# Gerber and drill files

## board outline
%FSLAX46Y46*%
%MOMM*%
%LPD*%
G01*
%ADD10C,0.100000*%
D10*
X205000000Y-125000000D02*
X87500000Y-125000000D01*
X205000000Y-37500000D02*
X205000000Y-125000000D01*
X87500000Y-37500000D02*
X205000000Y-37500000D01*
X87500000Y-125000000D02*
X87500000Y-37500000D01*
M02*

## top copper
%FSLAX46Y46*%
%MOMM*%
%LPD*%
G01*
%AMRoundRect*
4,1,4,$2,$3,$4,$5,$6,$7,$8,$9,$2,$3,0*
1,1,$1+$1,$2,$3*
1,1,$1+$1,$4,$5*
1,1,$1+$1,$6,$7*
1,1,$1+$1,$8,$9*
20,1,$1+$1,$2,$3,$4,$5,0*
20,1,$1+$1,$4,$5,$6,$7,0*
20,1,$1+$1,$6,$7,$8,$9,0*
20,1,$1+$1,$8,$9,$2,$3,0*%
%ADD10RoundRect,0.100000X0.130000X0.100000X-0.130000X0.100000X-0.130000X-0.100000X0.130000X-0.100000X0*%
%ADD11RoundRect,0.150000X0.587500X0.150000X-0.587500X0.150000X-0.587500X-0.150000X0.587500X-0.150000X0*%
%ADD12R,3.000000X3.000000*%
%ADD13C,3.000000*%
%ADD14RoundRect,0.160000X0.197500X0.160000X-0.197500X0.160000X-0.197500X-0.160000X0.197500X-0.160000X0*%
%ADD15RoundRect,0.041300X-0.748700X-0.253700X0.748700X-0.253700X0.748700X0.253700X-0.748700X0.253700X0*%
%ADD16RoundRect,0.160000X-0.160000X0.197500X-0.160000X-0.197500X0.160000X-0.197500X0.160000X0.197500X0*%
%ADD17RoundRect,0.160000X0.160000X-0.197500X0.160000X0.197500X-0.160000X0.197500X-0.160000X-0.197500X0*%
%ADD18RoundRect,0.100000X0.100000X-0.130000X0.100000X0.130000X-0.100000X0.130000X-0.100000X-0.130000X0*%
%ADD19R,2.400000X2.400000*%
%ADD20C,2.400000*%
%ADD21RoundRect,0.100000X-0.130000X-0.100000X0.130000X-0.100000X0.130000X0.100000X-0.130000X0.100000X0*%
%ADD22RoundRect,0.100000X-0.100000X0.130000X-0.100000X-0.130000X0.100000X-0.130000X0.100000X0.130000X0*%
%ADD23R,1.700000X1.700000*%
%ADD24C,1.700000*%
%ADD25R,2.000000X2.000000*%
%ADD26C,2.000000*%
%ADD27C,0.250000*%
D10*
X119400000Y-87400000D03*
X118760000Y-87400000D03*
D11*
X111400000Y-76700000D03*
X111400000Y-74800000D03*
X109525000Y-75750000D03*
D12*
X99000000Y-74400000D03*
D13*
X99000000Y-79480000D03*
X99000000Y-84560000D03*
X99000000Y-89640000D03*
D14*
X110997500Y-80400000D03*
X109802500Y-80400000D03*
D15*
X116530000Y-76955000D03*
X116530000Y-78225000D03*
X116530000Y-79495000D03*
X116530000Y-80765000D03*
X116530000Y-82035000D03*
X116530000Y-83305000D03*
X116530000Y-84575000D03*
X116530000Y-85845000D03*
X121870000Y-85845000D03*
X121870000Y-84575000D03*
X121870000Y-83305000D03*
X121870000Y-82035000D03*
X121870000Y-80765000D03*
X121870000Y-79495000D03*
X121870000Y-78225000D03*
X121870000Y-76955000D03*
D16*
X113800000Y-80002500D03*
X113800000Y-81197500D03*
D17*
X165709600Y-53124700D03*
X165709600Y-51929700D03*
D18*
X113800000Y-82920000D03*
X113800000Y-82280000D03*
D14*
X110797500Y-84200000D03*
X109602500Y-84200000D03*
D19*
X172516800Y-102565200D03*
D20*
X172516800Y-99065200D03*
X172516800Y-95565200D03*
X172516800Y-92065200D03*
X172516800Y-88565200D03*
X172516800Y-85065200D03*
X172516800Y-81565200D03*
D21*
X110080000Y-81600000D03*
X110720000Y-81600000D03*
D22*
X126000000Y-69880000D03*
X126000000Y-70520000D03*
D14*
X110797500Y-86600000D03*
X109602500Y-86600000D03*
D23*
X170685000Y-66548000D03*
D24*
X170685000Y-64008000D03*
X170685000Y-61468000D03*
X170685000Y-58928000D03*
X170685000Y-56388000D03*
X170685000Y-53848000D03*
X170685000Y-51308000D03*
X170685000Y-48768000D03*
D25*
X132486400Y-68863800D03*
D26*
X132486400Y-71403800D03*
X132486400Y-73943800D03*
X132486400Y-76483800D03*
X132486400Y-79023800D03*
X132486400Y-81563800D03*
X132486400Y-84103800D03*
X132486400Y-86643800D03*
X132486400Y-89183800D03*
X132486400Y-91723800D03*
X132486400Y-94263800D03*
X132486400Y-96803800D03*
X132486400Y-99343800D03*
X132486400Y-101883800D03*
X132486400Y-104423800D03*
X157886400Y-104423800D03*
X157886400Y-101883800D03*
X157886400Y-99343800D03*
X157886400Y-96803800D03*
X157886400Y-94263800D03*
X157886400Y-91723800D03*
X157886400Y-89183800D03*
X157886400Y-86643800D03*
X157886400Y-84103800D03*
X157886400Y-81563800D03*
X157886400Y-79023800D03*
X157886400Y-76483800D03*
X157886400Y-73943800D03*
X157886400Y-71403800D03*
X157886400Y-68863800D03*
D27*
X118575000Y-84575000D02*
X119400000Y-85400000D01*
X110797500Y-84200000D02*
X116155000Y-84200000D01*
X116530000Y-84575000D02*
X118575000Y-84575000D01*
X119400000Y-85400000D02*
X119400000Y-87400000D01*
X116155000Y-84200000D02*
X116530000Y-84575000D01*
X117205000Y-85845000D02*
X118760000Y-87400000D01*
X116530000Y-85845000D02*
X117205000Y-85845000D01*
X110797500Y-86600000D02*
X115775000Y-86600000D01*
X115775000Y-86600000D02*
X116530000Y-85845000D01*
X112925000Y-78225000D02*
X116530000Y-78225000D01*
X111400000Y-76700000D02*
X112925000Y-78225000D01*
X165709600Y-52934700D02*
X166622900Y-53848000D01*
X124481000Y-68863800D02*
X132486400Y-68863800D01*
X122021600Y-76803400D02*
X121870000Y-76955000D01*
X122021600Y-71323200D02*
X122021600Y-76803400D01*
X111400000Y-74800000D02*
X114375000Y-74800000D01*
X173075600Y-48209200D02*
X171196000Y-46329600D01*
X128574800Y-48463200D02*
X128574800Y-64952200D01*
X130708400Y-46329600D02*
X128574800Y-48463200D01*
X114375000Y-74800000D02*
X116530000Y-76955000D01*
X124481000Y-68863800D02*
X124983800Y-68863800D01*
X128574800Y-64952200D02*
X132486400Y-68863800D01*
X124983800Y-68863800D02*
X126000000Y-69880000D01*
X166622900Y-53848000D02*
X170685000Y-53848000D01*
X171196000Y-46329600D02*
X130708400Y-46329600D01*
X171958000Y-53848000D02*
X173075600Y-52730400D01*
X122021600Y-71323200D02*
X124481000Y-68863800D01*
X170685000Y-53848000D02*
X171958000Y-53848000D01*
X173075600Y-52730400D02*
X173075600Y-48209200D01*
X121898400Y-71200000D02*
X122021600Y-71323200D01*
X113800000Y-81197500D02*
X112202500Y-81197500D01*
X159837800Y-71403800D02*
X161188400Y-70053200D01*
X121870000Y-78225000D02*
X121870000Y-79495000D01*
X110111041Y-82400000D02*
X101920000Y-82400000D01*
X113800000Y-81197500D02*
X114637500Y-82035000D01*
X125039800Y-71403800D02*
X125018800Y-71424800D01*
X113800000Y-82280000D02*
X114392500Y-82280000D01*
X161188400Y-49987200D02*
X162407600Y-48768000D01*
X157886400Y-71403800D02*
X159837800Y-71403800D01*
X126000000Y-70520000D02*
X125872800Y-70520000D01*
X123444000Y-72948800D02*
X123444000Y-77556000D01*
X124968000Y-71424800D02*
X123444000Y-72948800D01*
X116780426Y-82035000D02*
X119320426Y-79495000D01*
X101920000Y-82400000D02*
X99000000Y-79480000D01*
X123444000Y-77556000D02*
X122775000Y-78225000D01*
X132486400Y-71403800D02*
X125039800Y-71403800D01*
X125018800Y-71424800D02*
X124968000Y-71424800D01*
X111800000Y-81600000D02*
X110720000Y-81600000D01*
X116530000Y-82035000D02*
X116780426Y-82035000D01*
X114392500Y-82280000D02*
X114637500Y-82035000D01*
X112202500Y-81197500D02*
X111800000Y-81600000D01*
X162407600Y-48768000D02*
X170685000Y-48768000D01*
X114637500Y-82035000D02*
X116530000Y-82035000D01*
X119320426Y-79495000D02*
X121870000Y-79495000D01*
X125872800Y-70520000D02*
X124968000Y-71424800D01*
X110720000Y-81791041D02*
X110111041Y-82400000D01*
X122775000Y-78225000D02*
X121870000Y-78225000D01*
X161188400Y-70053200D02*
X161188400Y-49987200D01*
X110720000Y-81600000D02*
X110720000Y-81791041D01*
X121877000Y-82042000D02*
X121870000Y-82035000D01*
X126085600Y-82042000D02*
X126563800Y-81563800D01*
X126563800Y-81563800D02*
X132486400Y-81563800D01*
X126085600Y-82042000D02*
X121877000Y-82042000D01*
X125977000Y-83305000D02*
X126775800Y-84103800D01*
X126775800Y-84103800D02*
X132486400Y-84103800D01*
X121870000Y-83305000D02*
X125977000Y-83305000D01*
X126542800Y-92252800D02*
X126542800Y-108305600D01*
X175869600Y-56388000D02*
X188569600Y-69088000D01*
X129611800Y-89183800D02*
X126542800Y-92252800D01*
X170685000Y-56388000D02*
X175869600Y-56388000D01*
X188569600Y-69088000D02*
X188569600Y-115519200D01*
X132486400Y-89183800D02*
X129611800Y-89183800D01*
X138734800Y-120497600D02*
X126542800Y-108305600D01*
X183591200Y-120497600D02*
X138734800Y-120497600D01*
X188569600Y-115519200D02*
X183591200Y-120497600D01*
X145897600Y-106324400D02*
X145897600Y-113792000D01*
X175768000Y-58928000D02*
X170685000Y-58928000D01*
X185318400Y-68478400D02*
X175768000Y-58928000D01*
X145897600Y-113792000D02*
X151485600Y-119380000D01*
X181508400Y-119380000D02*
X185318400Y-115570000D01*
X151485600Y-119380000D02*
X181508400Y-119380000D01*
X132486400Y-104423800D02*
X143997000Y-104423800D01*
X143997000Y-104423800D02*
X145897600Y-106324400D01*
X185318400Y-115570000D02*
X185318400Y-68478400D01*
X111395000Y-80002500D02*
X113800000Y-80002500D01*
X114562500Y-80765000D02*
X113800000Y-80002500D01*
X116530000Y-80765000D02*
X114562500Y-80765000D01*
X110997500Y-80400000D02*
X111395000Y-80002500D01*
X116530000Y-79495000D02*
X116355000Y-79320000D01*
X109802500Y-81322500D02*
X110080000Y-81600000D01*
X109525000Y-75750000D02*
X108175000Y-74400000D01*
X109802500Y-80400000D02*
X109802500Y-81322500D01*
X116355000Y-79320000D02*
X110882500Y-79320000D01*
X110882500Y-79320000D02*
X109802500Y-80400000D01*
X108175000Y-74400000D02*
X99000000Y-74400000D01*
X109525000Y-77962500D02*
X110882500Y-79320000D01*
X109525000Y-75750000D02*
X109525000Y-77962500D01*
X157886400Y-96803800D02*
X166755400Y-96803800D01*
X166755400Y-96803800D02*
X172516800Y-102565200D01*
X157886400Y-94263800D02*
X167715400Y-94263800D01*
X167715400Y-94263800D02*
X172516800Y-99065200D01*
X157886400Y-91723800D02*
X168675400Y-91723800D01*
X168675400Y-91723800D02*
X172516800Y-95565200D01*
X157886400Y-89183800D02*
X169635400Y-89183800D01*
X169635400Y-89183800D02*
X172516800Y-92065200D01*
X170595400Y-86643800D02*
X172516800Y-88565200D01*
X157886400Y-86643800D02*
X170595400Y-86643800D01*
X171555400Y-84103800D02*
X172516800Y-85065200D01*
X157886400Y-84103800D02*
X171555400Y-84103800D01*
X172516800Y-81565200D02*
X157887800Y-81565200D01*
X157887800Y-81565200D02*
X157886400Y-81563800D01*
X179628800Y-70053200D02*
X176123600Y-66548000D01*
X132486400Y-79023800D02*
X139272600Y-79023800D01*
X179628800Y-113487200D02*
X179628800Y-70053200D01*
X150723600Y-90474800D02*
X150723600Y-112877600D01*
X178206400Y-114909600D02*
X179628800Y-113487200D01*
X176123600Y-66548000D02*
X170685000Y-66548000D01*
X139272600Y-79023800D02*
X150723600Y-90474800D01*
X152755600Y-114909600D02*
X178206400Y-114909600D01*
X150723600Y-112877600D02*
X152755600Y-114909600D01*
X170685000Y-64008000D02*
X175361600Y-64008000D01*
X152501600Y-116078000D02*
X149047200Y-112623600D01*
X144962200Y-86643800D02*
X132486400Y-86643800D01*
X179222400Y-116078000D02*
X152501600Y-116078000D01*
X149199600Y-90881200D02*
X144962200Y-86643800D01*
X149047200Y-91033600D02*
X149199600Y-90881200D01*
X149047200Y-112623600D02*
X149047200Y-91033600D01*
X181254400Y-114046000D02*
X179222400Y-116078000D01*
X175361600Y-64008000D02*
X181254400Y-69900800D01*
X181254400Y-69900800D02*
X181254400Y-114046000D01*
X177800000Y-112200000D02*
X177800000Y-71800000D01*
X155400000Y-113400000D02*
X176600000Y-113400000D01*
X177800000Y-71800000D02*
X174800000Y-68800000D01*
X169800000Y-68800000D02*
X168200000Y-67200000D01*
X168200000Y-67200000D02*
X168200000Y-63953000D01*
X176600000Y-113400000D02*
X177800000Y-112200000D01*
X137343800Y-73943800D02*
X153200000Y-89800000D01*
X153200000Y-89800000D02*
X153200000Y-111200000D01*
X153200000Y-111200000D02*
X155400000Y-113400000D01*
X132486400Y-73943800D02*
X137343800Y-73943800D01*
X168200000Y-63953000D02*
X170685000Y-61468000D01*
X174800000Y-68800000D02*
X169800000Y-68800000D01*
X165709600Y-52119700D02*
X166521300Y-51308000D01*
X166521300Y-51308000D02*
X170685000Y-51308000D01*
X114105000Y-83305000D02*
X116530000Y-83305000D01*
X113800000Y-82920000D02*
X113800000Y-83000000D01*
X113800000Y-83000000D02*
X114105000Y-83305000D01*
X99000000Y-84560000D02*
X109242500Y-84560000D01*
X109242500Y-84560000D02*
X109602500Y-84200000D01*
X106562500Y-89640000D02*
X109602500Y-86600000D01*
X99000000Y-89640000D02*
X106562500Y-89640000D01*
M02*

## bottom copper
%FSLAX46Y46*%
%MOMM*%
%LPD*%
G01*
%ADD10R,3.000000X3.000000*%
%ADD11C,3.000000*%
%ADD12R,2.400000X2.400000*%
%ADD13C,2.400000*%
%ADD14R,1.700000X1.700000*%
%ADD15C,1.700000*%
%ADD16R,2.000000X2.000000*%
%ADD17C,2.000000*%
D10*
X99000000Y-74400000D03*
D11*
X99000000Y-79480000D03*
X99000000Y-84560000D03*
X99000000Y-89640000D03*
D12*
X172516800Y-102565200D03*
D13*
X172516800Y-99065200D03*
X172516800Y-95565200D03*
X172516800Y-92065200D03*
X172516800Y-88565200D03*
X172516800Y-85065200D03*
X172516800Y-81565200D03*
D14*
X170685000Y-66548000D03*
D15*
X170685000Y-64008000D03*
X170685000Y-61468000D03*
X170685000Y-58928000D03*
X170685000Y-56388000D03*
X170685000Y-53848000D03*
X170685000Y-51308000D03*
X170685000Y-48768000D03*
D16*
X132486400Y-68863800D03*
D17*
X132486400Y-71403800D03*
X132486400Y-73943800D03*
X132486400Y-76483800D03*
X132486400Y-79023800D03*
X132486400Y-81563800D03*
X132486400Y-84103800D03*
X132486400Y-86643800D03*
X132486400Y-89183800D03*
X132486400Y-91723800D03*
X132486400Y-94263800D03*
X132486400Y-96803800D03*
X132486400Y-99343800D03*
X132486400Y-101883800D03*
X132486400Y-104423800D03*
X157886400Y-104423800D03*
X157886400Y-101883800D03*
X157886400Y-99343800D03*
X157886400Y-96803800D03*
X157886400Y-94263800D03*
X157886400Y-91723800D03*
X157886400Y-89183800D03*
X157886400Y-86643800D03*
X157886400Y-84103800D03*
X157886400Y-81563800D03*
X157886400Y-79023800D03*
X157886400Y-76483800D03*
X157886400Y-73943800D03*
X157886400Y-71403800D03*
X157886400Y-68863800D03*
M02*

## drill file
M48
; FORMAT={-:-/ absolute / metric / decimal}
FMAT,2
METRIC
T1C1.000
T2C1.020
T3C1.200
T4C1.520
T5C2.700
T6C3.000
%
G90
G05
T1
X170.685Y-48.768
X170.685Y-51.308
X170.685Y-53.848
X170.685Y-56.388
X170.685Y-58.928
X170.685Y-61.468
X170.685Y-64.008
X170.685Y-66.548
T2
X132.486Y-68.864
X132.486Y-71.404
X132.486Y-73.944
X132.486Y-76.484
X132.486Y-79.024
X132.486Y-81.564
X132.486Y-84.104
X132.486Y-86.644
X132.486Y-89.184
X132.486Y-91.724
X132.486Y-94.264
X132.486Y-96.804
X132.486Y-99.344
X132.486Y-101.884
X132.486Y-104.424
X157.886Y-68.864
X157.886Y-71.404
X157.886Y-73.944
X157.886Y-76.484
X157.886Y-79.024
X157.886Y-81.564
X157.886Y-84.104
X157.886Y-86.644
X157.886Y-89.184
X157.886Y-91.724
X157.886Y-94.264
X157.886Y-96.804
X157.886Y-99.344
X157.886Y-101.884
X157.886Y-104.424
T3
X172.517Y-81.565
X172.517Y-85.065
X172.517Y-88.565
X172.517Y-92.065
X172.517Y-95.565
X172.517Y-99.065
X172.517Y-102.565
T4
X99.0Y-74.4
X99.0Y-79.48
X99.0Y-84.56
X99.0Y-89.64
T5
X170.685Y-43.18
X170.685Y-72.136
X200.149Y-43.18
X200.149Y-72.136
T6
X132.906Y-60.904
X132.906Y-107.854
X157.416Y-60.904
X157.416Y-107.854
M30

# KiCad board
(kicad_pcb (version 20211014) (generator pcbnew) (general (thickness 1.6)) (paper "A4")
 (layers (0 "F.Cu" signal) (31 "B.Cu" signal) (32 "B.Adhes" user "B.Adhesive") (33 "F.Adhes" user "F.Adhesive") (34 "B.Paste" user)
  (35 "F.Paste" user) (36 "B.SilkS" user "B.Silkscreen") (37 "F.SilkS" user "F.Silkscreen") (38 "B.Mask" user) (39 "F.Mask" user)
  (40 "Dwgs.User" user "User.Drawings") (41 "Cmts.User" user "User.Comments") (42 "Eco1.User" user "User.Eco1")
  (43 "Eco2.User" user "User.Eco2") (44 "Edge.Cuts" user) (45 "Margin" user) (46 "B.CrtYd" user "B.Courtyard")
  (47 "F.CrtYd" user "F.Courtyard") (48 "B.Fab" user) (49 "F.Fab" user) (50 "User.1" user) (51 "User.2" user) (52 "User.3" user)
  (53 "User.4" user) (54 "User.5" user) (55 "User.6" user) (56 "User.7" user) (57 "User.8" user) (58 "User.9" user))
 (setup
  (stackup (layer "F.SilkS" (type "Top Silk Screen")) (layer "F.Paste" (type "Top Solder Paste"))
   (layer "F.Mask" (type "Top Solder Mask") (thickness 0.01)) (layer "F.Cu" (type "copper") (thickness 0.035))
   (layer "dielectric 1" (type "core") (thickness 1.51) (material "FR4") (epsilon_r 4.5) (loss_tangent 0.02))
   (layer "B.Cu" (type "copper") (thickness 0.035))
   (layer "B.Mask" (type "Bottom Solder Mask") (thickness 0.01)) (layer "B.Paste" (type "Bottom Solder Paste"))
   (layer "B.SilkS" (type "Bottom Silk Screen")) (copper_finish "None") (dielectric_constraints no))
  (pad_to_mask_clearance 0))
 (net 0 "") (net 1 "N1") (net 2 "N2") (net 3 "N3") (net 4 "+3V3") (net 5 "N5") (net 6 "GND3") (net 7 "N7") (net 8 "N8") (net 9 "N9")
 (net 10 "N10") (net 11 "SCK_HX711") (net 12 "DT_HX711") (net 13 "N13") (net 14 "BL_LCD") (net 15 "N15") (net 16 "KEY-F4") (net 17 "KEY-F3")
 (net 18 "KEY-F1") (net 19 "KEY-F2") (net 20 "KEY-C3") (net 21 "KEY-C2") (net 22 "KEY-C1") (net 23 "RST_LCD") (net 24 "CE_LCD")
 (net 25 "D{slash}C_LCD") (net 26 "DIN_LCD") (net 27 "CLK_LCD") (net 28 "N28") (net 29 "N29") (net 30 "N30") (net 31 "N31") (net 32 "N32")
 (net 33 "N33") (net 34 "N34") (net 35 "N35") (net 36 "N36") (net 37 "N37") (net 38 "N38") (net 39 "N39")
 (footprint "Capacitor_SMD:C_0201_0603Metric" (layer "F.Cu") (at 119.08 87.4 180)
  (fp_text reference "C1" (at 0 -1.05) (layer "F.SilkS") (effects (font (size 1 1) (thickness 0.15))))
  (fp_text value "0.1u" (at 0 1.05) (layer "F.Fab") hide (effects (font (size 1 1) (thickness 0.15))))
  (pad "" smd roundrect (at 0.345 0 180) (size 0.318 0.36) (layers "F.Paste") (roundrect_rratio 0.25))
  (pad "" smd roundrect (at -0.345 0 180) (size 0.318 0.36) (layers "F.Paste") (roundrect_rratio 0.25))
  (pad "1" smd roundrect (at -0.32 0 180) (size 0.46 0.4) (layers "F.Cu" "F.Mask") (roundrect_rratio 0.25) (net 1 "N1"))
  (pad "2" smd roundrect (at 0.32 0 180) (size 0.46 0.4) (layers "F.Cu" "F.Mask") (roundrect_rratio 0.25) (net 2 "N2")))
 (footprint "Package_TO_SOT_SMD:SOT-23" (layer "F.Cu") (at 110.4625 75.75 180)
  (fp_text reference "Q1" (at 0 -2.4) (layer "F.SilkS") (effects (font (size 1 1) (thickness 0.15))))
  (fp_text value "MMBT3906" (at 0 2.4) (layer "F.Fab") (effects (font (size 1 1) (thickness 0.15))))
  (pad "1" smd roundrect (at -0.9375 -0.95 180) (size 1.475 0.6) (layers "F.Cu" "F.Paste" "F.Mask") (roundrect_rratio 0.25) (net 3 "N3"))
  (pad "2" smd roundrect (at -0.9375 0.95 180) (size 1.475 0.6) (layers "F.Cu" "F.Paste" "F.Mask") (roundrect_rratio 0.25) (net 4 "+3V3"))
  (pad "3" smd roundrect (at 0.9375 0 180) (size 1.475 0.6) (layers "F.Cu" "F.Paste" "F.Mask") (roundrect_rratio 0.25) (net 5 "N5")))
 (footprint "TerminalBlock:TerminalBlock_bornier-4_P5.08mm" (layer "F.Cu") (at 99 74.4 -90)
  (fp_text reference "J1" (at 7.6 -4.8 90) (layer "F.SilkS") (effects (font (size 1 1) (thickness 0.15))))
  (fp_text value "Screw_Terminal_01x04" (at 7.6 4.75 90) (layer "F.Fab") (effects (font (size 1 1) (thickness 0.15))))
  (pad "1" thru_hole rect (at 0 0 270) (size 3 3) (drill 1.52) (layers *.Cu *.Mask) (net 5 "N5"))
  (pad "2" thru_hole circle (at 5.08 0 270) (size 3 3) (drill 1.52) (layers *.Cu *.Mask) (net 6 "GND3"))
  (pad "3" thru_hole circle (at 10.16 0 270) (size 3 3) (drill 1.52) (layers *.Cu *.Mask) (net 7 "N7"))
  (pad "4" thru_hole circle (at 15.24 0 270) (size 3 3) (drill 1.52) (layers *.Cu *.Mask) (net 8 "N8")))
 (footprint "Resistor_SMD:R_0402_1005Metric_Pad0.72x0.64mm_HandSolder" (layer "F.Cu") (at 110.4 80.4 180)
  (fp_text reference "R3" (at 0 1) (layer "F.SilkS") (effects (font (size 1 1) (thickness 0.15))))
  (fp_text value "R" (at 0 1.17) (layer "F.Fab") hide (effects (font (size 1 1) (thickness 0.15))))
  (pad "1" smd roundrect (at -0.5975 0 180) (size 0.715 0.64) (layers "F.Cu" "F.Paste" "F.Mask") (roundrect_rratio 0.25) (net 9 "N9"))
  (pad "2" smd roundrect (at 0.5975 0 180) (size 0.715 0.64) (layers "F.Cu" "F.Paste" "F.Mask") (roundrect_rratio 0.25) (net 5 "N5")))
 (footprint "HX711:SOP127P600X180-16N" (layer "F.Cu") (at 119.2 81.4)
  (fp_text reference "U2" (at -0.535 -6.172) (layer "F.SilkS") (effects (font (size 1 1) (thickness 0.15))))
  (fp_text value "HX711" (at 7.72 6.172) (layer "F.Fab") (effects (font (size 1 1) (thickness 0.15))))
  (pad "1" smd roundrect locked (at -2.67 -4.445) (size 1.58 0.59) (layers "F.Cu" "F.Paste" "F.Mask") (roundrect_rratio 0.07) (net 4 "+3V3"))
  (pad "2" smd roundrect locked (at -2.67 -3.175) (size 1.58 0.59) (layers "F.Cu" "F.Paste" "F.Mask") (roundrect_rratio 0.07) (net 3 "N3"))
  (pad "3" smd roundrect locked (at -2.67 -1.905) (size 1.58 0.59) (layers "F.Cu" "F.Paste" "F.Mask") (roundrect_rratio 0.07) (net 5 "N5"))
  (pad "4" smd roundrect locked (at -2.67 -0.635) (size 1.58 0.59) (layers "F.Cu" "F.Paste" "F.Mask") (roundrect_rratio 0.07) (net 9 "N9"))
  (pad "5" smd roundrect locked (at -2.67 0.635) (size 1.58 0.59) (layers "F.Cu" "F.Paste" "F.Mask") (roundrect_rratio 0.07) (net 6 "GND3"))
  (pad "6" smd roundrect locked (at -2.67 1.905) (size 1.58 0.59) (layers "F.Cu" "F.Paste" "F.Mask") (roundrect_rratio 0.07) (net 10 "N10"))
  (pad "7" smd roundrect locked (at -2.67 3.175) (size 1.58 0.59) (layers "F.Cu" "F.Paste" "F.Mask") (roundrect_rratio 0.07) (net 1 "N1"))
  (pad "8" smd roundrect locked (at -2.67 4.445) (size 1.58 0.59) (layers "F.Cu" "F.Paste" "F.Mask") (roundrect_rratio 0.07) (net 2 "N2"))
  (pad "9" smd roundrect locked (at 2.67 4.445) (size 1.58 0.59) (layers "F.Cu" "F.Paste" "F.Mask") (roundrect_rratio 0.07) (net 6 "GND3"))
  (pad "10" smd roundrect locked (at 2.67 3.175) (size 1.58 0.59) (layers "F.Cu" "F.Paste" "F.Mask") (roundrect_rratio 0.07) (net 4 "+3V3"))
  (pad "11" smd roundrect locked (at 2.67 1.905) (size 1.58 0.59) (layers "F.Cu" "F.Paste" "F.Mask") (roundrect_rratio 0.07)
   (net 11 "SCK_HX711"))
  (pad "12" smd roundrect locked (at 2.67 0.635) (size 1.58 0.59) (layers "F.Cu" "F.Paste" "F.Mask") (roundrect_rratio 0.07)
   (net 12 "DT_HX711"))
  (pad "13" smd roundrect locked (at 2.67 -0.635) (size 1.58 0.59) (layers "F.Cu" "F.Paste" "F.Mask") (roundrect_rratio 0.07) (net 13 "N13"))
  (pad "14" smd roundrect locked (at 2.67 -1.905) (size 1.58 0.59) (layers "F.Cu" "F.Paste" "F.Mask") (roundrect_rratio 0.07) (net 6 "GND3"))
  (pad "15" smd roundrect locked (at 2.67 -3.175) (size 1.58 0.59) (layers "F.Cu" "F.Paste" "F.Mask") (roundrect_rratio 0.07) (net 6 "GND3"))
  (pad "16" smd roundrect locked (at 2.67 -4.445) (size 1.58 0.59) (layers "F.Cu" "F.Paste" "F.Mask") (roundrect_rratio 0.07) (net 4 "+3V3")))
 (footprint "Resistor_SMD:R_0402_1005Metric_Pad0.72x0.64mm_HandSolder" (layer "F.Cu") (at 113.8 80.6 -90)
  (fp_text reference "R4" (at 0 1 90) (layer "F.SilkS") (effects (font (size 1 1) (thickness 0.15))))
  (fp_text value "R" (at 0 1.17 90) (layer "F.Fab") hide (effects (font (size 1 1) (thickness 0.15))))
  (pad "1" smd roundrect (at -0.5975 0 270) (size 0.715 0.64) (layers "F.Cu" "F.Paste" "F.Mask") (roundrect_rratio 0.25) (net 9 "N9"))
  (pad "2" smd roundrect (at 0.5975 0 270) (size 0.715 0.64) (layers "F.Cu" "F.Paste" "F.Mask") (roundrect_rratio 0.25) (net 6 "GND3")))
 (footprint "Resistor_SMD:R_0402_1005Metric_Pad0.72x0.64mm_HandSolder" (layer "F.Cu") (at 165.7096 52.5272 90)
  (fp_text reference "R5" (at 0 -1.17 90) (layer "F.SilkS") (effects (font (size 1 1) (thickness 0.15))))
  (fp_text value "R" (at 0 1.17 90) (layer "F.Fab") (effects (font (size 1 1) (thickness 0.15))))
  (pad "1" smd roundrect (at -0.5975 0 90) (size 0.715 0.64) (layers "F.Cu" "F.Paste" "F.Mask") (roundrect_rratio 0.25) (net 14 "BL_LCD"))
  (pad "2" smd roundrect (at 0.5975 0 90) (size 0.715 0.64) (layers "F.Cu" "F.Paste" "F.Mask") (roundrect_rratio 0.25) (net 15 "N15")))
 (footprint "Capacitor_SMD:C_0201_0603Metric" (layer "F.Cu") (at 113.8 82.6 90)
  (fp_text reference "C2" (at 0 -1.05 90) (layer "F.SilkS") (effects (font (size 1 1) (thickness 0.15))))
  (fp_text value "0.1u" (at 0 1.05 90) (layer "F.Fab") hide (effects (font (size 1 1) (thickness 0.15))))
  (pad "" smd roundrect (at -0.345 0 90) (size 0.318 0.36) (layers "F.Paste") (roundrect_rratio 0.25))
  (pad "" smd roundrect (at 0.345 0 90) (size 0.318 0.36) (layers "F.Paste") (roundrect_rratio 0.25))
  (pad "1" smd roundrect (at -0.32 0 90) (size 0.46 0.4) (layers "F.Cu" "F.Mask") (roundrect_rratio 0.25) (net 10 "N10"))
  (pad "2" smd roundrect (at 0.32 0 90) (size 0.46 0.4) (layers "F.Cu" "F.Mask") (roundrect_rratio 0.25) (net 6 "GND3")))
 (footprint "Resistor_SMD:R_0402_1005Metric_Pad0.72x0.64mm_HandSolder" (layer "F.Cu") (at 110.2 84.2 180)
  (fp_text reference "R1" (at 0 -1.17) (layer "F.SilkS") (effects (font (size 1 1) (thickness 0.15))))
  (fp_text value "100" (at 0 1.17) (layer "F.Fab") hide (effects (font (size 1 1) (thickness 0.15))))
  (pad "1" smd roundrect (at -0.5975 0 180) (size 0.715 0.64) (layers "F.Cu" "F.Paste" "F.Mask") (roundrect_rratio 0.25) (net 1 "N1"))
  (pad "2" smd roundrect (at 0.5975 0 180) (size 0.715 0.64) (layers "F.Cu" "F.Paste" "F.Mask") (roundrect_rratio 0.25) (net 7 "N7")))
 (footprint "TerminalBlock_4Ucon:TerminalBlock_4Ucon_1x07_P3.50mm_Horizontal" (layer "F.Cu") (at 172.5168 102.5652 90)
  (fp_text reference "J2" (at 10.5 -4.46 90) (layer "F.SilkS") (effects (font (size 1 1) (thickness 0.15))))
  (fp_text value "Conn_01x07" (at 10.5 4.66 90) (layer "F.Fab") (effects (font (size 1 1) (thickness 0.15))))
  (pad "1" thru_hole rect (at 0 0 90) (size 2.4 2.4) (drill 1.2) (layers *.Cu *.Mask) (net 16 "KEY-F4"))
  (pad "2" thru_hole circle (at 3.5 0 90) (size 2.4 2.4) (drill 1.2) (layers *.Cu *.Mask) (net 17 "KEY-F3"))
  (pad "3" thru_hole circle (at 7 0 90) (size 2.4 2.4) (drill 1.2) (layers *.Cu *.Mask) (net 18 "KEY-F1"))
  (pad "4" thru_hole circle (at 10.5 0 90) (size 2.4 2.4) (drill 1.2) (layers *.Cu *.Mask) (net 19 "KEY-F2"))
  (pad "5" thru_hole circle (at 14 0 90) (size 2.4 2.4) (drill 1.2) (layers *.Cu *.Mask) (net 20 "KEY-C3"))
  (pad "6" thru_hole circle (at 17.5 0 90) (size 2.4 2.4) (drill 1.2) (layers *.Cu *.Mask) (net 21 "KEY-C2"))
  (pad "7" thru_hole circle (at 21 0 90) (size 2.4 2.4) (drill 1.2) (layers *.Cu *.Mask) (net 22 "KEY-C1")))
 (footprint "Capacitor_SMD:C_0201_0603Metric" (layer "F.Cu") (at 110.4 81.6)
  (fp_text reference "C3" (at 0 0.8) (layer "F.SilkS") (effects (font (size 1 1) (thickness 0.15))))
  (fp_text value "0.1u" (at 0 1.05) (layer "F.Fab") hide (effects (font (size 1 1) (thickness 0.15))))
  (pad "" smd roundrect (at -0.345 0) (size 0.318 0.36) (layers "F.Paste") (roundrect_rratio 0.25))
  (pad "" smd roundrect (at 0.345 0) (size 0.318 0.36) (layers "F.Paste") (roundrect_rratio 0.25))
  (pad "1" smd roundrect (at -0.32 0) (size 0.46 0.4) (layers "F.Cu" "F.Mask") (roundrect_rratio 0.25) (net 5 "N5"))
  (pad "2" smd roundrect (at 0.32 0) (size 0.46 0.4) (layers "F.Cu" "F.Mask") (roundrect_rratio 0.25) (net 6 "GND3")))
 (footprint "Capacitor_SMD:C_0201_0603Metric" (layer "F.Cu") (at 126 70.2 -90)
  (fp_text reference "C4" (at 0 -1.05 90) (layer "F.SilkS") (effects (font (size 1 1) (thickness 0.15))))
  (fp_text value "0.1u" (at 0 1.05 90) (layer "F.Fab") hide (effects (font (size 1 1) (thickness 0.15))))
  (pad "" smd roundrect (at -0.345 0 270) (size 0.318 0.36) (layers "F.Paste") (roundrect_rratio 0.25))
  (pad "" smd roundrect (at 0.345 0 270) (size 0.318 0.36) (layers "F.Paste") (roundrect_rratio 0.25))
  (pad "1" smd roundrect (at -0.32 0 270) (size 0.46 0.4) (layers "F.Cu" "F.Mask") (roundrect_rratio 0.25) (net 4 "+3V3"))
  (pad "2" smd roundrect (at 0.32 0 270) (size 0.46 0.4) (layers "F.Cu" "F.Mask") (roundrect_rratio 0.25) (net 6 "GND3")))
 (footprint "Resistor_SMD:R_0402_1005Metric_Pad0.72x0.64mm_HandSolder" (layer "F.Cu") (at 110.2 86.6 180)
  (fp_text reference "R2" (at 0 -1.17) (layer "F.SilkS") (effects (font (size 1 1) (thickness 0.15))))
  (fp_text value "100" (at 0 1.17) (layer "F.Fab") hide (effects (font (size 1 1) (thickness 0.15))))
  (pad "1" smd roundrect (at -0.5975 0 180) (size 0.715 0.64) (layers "F.Cu" "F.Paste" "F.Mask") (roundrect_rratio 0.25) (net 2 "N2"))
  (pad "2" smd roundrect (at 0.5975 0 180) (size 0.715 0.64) (layers "F.Cu" "F.Paste" "F.Mask") (roundrect_rratio 0.25) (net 8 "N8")))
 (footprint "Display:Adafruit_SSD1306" (layer "F.Cu") (at 170.685 66.548 90)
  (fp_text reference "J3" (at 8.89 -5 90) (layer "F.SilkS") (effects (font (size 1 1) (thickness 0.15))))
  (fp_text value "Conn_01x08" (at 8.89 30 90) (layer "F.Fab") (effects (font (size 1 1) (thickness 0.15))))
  (pad "" np_thru_hole circle (at 23.368 29.464 90) (size 2.7 2.7) (drill 2.7) (layers *.Cu *.Mask))
  (pad "" np_thru_hole circle (at -5.588 0 90) (size 2.7 2.7) (drill 2.7) (layers *.Cu *.Mask))
  (pad "" np_thru_hole circle (at -5.588 29.464 90) (size 2.7 2.7) (drill 2.7) (layers *.Cu *.Mask))
  (pad "" np_thru_hole circle (at 23.368 0 90) (size 2.7 2.7) (drill 2.7) (layers *.Cu *.Mask))
  (pad "1" thru_hole rect (at 0 0 90) (size 1.7 1.7) (drill 1) (layers *.Cu *.Mask) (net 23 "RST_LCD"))
  (pad "2" thru_hole circle (at 2.54 0 90) (size 1.7 1.7) (drill 1) (layers *.Cu *.Mask) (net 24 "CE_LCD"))
  (pad "3" thru_hole circle (at 5.08 0 90) (size 1.7 1.7) (drill 1) (layers *.Cu *.Mask) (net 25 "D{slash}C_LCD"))
  (pad "4" thru_hole circle (at 7.62 0 90) (size 1.7 1.7) (drill 1) (layers *.Cu *.Mask) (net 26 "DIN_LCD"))
  (pad "5" thru_hole circle (at 10.16 0 90) (size 1.7 1.7) (drill 1) (layers *.Cu *.Mask) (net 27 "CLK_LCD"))
  (pad "6" thru_hole circle (at 12.7 0 90) (size 1.7 1.7) (drill 1) (layers *.Cu *.Mask) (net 4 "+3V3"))
  (pad "7" thru_hole circle (at 15.24 0 90) (size 1.7 1.7) (drill 1) (layers *.Cu *.Mask) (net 15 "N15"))
  (pad "8" thru_hole circle (at 17.78 0 90) (size 1.7 1.7) (drill 1) (layers *.Cu *.Mask) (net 6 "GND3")))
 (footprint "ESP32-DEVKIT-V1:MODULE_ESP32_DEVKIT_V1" (layer "F.Cu") (at 145.1864 84.3788)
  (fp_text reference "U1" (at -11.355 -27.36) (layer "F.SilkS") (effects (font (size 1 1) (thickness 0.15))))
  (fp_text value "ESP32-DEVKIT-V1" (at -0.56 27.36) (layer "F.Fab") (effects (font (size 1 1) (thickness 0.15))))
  (pad "" np_thru_hole circle locked (at -12.28 -23.475) (size 3 3) (drill 3) (layers *.Cu *.Mask))
  (pad "" np_thru_hole circle locked (at -12.28 23.475) (size 3 3) (drill 3) (layers *.Cu *.Mask))
  (pad "" np_thru_hole circle locked (at 12.23 -23.475) (size 3 3) (drill 3) (layers *.Cu *.Mask))
  (pad "" np_thru_hole circle locked (at 12.23 23.475) (size 3 3) (drill 3) (layers *.Cu *.Mask))
  (pad "1" thru_hole rect locked (at -12.7 -15.515) (size 2 2) (drill 1.02) (layers *.Cu *.Mask) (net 4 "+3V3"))
  (pad "2" thru_hole circle locked (at -12.7 -12.975) (size 2 2) (drill 1.02) (layers *.Cu *.Mask) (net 6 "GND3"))
  (pad "3" thru_hole circle locked (at -12.7 -10.435) (size 2 2) (drill 1.02) (layers *.Cu *.Mask) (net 25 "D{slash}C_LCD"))
  (pad "4" thru_hole circle locked (at -12.7 -7.895) (size 2 2) (drill 1.02) (layers *.Cu *.Mask) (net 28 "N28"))
  (pad "5" thru_hole circle locked (at -12.7 -5.355) (size 2 2) (drill 1.02) (layers *.Cu *.Mask) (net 23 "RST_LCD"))
  (pad "6" thru_hole circle locked (at -12.7 -2.815) (size 2 2) (drill 1.02) (layers *.Cu *.Mask) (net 12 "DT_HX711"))
  (pad "7" thru_hole circle locked (at -12.7 -0.275) (size 2 2) (drill 1.02) (layers *.Cu *.Mask) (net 11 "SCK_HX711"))
  (pad "8" thru_hole circle locked (at -12.7 2.265) (size 2 2) (drill 1.02) (layers *.Cu *.Mask) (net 24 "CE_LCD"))
  (pad "9" thru_hole circle locked (at -12.7 4.805) (size 2 2) (drill 1.02) (layers *.Cu *.Mask) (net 27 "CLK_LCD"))
  (pad "10" thru_hole circle locked (at -12.7 7.345) (size 2 2) (drill 1.02) (layers *.Cu *.Mask) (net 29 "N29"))
  (pad "11" thru_hole circle locked (at -12.7 9.885) (size 2 2) (drill 1.02) (layers *.Cu *.Mask) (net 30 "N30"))
  (pad "12" thru_hole circle locked (at -12.7 12.425) (size 2 2) (drill 1.02) (layers *.Cu *.Mask) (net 14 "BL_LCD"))
  (pad "13" thru_hole circle locked (at -12.7 14.965) (size 2 2) (drill 1.02) (layers *.Cu *.Mask) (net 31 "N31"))
  (pad "14" thru_hole circle locked (at -12.7 17.505) (size 2 2) (drill 1.02) (layers *.Cu *.Mask) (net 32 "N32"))
  (pad "15" thru_hole circle locked (at -12.7 20.045) (size 2 2) (drill 1.02) (layers *.Cu *.Mask) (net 26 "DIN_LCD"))
  (pad "16" thru_hole circle locked (at 12.7 20.045) (size 2 2) (drill 1.02) (layers *.Cu *.Mask) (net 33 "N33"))
  (pad "17" thru_hole circle locked (at 12.7 17.505) (size 2 2) (drill 1.02) (layers *.Cu *.Mask) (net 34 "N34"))
  (pad "18" thru_hole circle locked (at 12.7 14.965) (size 2 2) (drill 1.02) (layers *.Cu *.Mask) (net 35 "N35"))
  (pad "19" thru_hole circle locked (at 12.7 12.425) (size 2 2) (drill 1.02) (layers *.Cu *.Mask) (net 16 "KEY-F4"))
  (pad "20" thru_hole circle locked (at 12.7 9.885) (size 2 2) (drill 1.02) (layers *.Cu *.Mask) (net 17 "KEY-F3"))
  (pad "21" thru_hole circle locked (at 12.7 7.345) (size 2 2) (drill 1.02) (layers *.Cu *.Mask) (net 18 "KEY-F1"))
  (pad "22" thru_hole circle locked (at 12.7 4.805) (size 2 2) (drill 1.02) (layers *.Cu *.Mask) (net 19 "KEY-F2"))
  (pad "23" thru_hole circle locked (at 12.7 2.265) (size 2 2) (drill 1.02) (layers *.Cu *.Mask) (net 20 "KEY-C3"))
  (pad "24" thru_hole circle locked (at 12.7 -0.275) (size 2 2) (drill 1.02) (layers *.Cu *.Mask) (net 21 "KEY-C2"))
  (pad "25" thru_hole circle locked (at 12.7 -2.815) (size 2 2) (drill 1.02) (layers *.Cu *.Mask) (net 22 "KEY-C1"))
  (pad "26" thru_hole circle locked (at 12.7 -5.355) (size 2 2) (drill 1.02) (layers *.Cu *.Mask) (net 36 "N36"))
  (pad "27" thru_hole circle locked (at 12.7 -7.895) (size 2 2) (drill 1.02) (layers *.Cu *.Mask) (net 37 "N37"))
  (pad "28" thru_hole circle locked (at 12.7 -10.435) (size 2 2) (drill 1.02) (layers *.Cu *.Mask) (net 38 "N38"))
  (pad "29" thru_hole circle locked (at 12.7 -12.975) (size 2 2) (drill 1.02) (layers *.Cu *.Mask) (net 6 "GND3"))
  (pad "30" thru_hole circle locked (at 12.7 -15.515) (size 2 2) (drill 1.02) (layers *.Cu *.Mask) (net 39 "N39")))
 (gr_line (start 205 125) (end 87.5 125) (layer "Edge.Cuts") (width 0.1))
 (gr_line (start 205 37.5) (end 205 125) (layer "Edge.Cuts") (width 0.1))
 (gr_line (start 87.5 37.5) (end 205 37.5) (layer "Edge.Cuts") (width 0.1))
 (gr_line (start 87.5 125) (end 87.5 37.5) (layer "Edge.Cuts") (width 0.1))
 (segment (start 118.575 84.575) (end 119.4 85.4) (width 0.25) (layer "F.Cu") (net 1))
 (segment (start 110.7975 84.2) (end 116.155 84.2) (width 0.25) (layer "F.Cu") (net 1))
 (segment (start 116.53 84.575) (end 118.575 84.575) (width 0.25) (layer "F.Cu") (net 1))
 (segment (start 119.4 85.4) (end 119.4 87.4) (width 0.25) (layer "F.Cu") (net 1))
 (segment (start 116.155 84.2) (end 116.53 84.575) (width 0.25) (layer "F.Cu") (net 1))
 (segment (start 117.205 85.845) (end 118.76 87.4) (width 0.25) (layer "F.Cu") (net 2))
 (segment (start 116.53 85.845) (end 117.205 85.845) (width 0.25) (layer "F.Cu") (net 2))
 (segment (start 110.7975 86.6) (end 115.775 86.6) (width 0.25) (layer "F.Cu") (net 2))
 (segment (start 115.775 86.6) (end 116.53 85.845) (width 0.25) (layer "F.Cu") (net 2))
 (segment (start 112.925 78.225) (end 116.53 78.225) (width 0.25) (layer "F.Cu") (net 3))
 (segment (start 111.4 76.7) (end 112.925 78.225) (width 0.25) (layer "F.Cu") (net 3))
 (segment (start 165.7096 52.9347) (end 166.6229 53.848) (width 0.25) (layer "F.Cu") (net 4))
 (segment (start 124.481 68.8638) (end 132.4864 68.8638) (width 0.25) (layer "F.Cu") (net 4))
 (segment (start 122.0216 76.8034) (end 121.87 76.955) (width 0.25) (layer "F.Cu") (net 4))
 (segment (start 122.0216 71.3232) (end 122.0216 76.8034) (width 0.25) (layer "F.Cu") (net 4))
 (segment (start 111.4 74.8) (end 114.375 74.8) (width 0.25) (layer "F.Cu") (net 4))
 (segment (start 173.0756 48.2092) (end 171.196 46.3296) (width 0.25) (layer "F.Cu") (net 4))
 (segment (start 128.5748 48.4632) (end 128.5748 64.9522) (width 0.25) (layer "F.Cu") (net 4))
 (segment (start 130.7084 46.3296) (end 128.5748 48.4632) (width 0.25) (layer "F.Cu") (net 4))
 (segment (start 114.375 74.8) (end 116.53 76.955) (width 0.25) (layer "F.Cu") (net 4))
 (segment (start 124.481 68.8638) (end 124.9838 68.8638) (width 0.25) (layer "F.Cu") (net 4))
 (segment (start 128.5748 64.9522) (end 132.4864 68.8638) (width 0.25) (layer "F.Cu") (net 4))
 (segment (start 124.9838 68.8638) (end 126 69.88) (width 0.25) (layer "F.Cu") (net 4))
 (segment (start 166.6229 53.848) (end 170.685 53.848) (width 0.25) (layer "F.Cu") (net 4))
 (segment (start 171.196 46.3296) (end 130.7084 46.3296) (width 0.25) (layer "F.Cu") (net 4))
 (segment (start 171.958 53.848) (end 173.0756 52.7304) (width 0.25) (layer "F.Cu") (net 4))
 (segment (start 122.0216 71.3232) (end 124.481 68.8638) (width 0.25) (layer "F.Cu") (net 4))
 (segment (start 170.685 53.848) (end 171.958 53.848) (width 0.25) (layer "F.Cu") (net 4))
 (segment (start 173.0756 52.7304) (end 173.0756 48.2092) (width 0.25) (layer "F.Cu") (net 4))
 (segment (start 121.8984 71.2) (end 122.0216 71.3232) (width 0.25) (layer "F.Cu") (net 4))
 (segment (start 113.8 81.1975) (end 112.2025 81.1975) (width 0.25) (layer "F.Cu") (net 6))
 (segment (start 159.8378 71.4038) (end 161.1884 70.0532) (width 0.25) (layer "F.Cu") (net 6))
 (segment (start 121.87 78.225) (end 121.87 79.495) (width 0.25) (layer "F.Cu") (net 6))
 (segment (start 110.111041 82.4) (end 101.92 82.4) (width 0.25) (layer "F.Cu") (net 6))
 (segment (start 113.8 81.1975) (end 114.6375 82.035) (width 0.25) (layer "F.Cu") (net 6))
 (segment (start 125.0398 71.4038) (end 125.0188 71.4248) (width 0.25) (layer "F.Cu") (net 6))
 (segment (start 113.8 82.28) (end 114.3925 82.28) (width 0.25) (layer "F.Cu") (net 6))
 (segment (start 161.1884 49.9872) (end 162.4076 48.768) (width 0.25) (layer "F.Cu") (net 6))
 (segment (start 157.8864 71.4038) (end 159.8378 71.4038) (width 0.25) (layer "F.Cu") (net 6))
 (segment (start 126 70.52) (end 125.8728 70.52) (width 0.25) (layer "F.Cu") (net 6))
 (segment (start 123.444 72.9488) (end 123.444 77.556) (width 0.25) (layer "F.Cu") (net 6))
 (segment (start 124.968 71.4248) (end 123.444 72.9488) (width 0.25) (layer "F.Cu") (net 6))
 (segment (start 116.780426 82.035) (end 119.320426 79.495) (width 0.25) (layer "F.Cu") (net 6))
 (segment (start 101.92 82.4) (end 99 79.48) (width 0.25) (layer "F.Cu") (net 6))
 (segment (start 123.444 77.556) (end 122.775 78.225) (width 0.25) (layer "F.Cu") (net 6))
 (segment (start 132.4864 71.4038) (end 125.0398 71.4038) (width 0.25) (layer "F.Cu") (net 6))
 (segment (start 125.0188 71.4248) (end 124.968 71.4248) (width 0.25) (layer "F.Cu") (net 6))
 (segment (start 111.8 81.6) (end 110.72 81.6) (width 0.25) (layer "F.Cu") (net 6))
 (segment (start 116.53 82.035) (end 116.780426 82.035) (width 0.25) (layer "F.Cu") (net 6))
 (segment (start 114.3925 82.28) (end 114.6375 82.035) (width 0.25) (layer "F.Cu") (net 6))
 (segment (start 112.2025 81.1975) (end 111.8 81.6) (width 0.25) (layer "F.Cu") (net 6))
 (segment (start 162.4076 48.768) (end 170.685 48.768) (width 0.25) (layer "F.Cu") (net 6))
 (segment (start 114.6375 82.035) (end 116.53 82.035) (width 0.25) (layer "F.Cu") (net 6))
 (segment (start 119.320426 79.495) (end 121.87 79.495) (width 0.25) (layer "F.Cu") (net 6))
 (segment (start 125.8728 70.52) (end 124.968 71.4248) (width 0.25) (layer "F.Cu") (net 6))
 (segment (start 110.72 81.791041) (end 110.111041 82.4) (width 0.25) (layer "F.Cu") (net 6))
 (segment (start 122.775 78.225) (end 121.87 78.225) (width 0.25) (layer "F.Cu") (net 6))
 (segment (start 161.1884 70.0532) (end 161.1884 49.9872) (width 0.25) (layer "F.Cu") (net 6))
 (segment (start 110.72 81.6) (end 110.72 81.791041) (width 0.25) (layer "F.Cu") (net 6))
 (segment (start 121.877 82.042) (end 121.87 82.035) (width 0.25) (layer "F.Cu") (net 12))
 (segment (start 126.0856 82.042) (end 126.5638 81.5638) (width 0.25) (layer "F.Cu") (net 12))
 (segment (start 126.5638 81.5638) (end 132.4864 81.5638) (width 0.25) (layer "F.Cu") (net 12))
 (segment (start 126.0856 82.042) (end 121.877 82.042) (width 0.25) (layer "F.Cu") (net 12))
 (segment (start 125.977 83.305) (end 126.7758 84.1038) (width 0.25) (layer "F.Cu") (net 11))
 (segment (start 126.7758 84.1038) (end 132.4864 84.1038) (width 0.25) (layer "F.Cu") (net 11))
 (segment (start 121.87 83.305) (end 125.977 83.305) (width 0.25) (layer "F.Cu") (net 11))
 (segment (start 126.5428 92.2528) (end 126.5428 108.3056) (width 0.25) (layer "F.Cu") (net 27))
 (segment (start 175.8696 56.388) (end 188.5696 69.088) (width 0.25) (layer "F.Cu") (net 27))
 (segment (start 129.6118 89.1838) (end 126.5428 92.2528) (width 0.25) (layer "F.Cu") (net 27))
 (segment (start 170.685 56.388) (end 175.8696 56.388) (width 0.25) (layer "F.Cu") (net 27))
 (segment (start 188.5696 69.088) (end 188.5696 115.5192) (width 0.25) (layer "F.Cu") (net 27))
 (segment (start 132.4864 89.1838) (end 129.6118 89.1838) (width 0.25) (layer "F.Cu") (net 27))
 (segment (start 138.7348 120.4976) (end 126.5428 108.3056) (width 0.25) (layer "F.Cu") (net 27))
 (segment (start 183.5912 120.4976) (end 138.7348 120.4976) (width 0.25) (layer "F.Cu") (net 27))
 (segment (start 188.5696 115.5192) (end 183.5912 120.4976) (width 0.25) (layer "F.Cu") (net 27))
 (segment (start 145.8976 106.3244) (end 145.8976 113.792) (width 0.25) (layer "F.Cu") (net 26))
 (segment (start 175.768 58.928) (end 170.685 58.928) (width 0.25) (layer "F.Cu") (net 26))
 (segment (start 185.3184 68.4784) (end 175.768 58.928) (width 0.25) (layer "F.Cu") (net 26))
 (segment (start 145.8976 113.792) (end 151.4856 119.38) (width 0.25) (layer "F.Cu") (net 26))
 (segment (start 181.5084 119.38) (end 185.3184 115.57) (width 0.25) (layer "F.Cu") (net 26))
 (segment (start 151.4856 119.38) (end 181.5084 119.38) (width 0.25) (layer "F.Cu") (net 26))
 (segment (start 132.4864 104.4238) (end 143.997 104.4238) (width 0.25) (layer "F.Cu") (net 26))
 (segment (start 143.997 104.4238) (end 145.8976 106.3244) (width 0.25) (layer "F.Cu") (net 26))
 (segment (start 185.3184 115.57) (end 185.3184 68.4784) (width 0.25) (layer "F.Cu") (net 26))
 (segment (start 111.395 80.0025) (end 113.8 80.0025) (width 0.25) (layer "F.Cu") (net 9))
 (segment (start 114.5625 80.765) (end 113.8 80.0025) (width 0.25) (layer "F.Cu") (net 9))
 (segment (start 116.53 80.765) (end 114.5625 80.765) (width 0.25) (layer "F.Cu") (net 9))
 (segment (start 110.9975 80.4) (end 111.395 80.0025) (width 0.25) (layer "F.Cu") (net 9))
 (segment (start 116.53 79.495) (end 116.355 79.32) (width 0.25) (layer "F.Cu") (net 5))
 (segment (start 109.8025 81.3225) (end 110.08 81.6) (width 0.25) (layer "F.Cu") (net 5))
 (segment (start 109.525 75.75) (end 108.175 74.4) (width 0.25) (layer "F.Cu") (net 5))
 (segment (start 109.8025 80.4) (end 109.8025 81.3225) (width 0.25) (layer "F.Cu") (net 5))
 (segment (start 116.355 79.32) (end 110.8825 79.32) (width 0.25) (layer "F.Cu") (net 5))
 (segment (start 110.8825 79.32) (end 109.8025 80.4) (width 0.25) (layer "F.Cu") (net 5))
 (segment (start 108.175 74.4) (end 99 74.4) (width 0.25) (layer "F.Cu") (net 5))
 (segment (start 109.525 77.9625) (end 110.8825 79.32) (width 0.25) (layer "F.Cu") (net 5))
 (segment (start 109.525 75.75) (end 109.525 77.9625) (width 0.25) (layer "F.Cu") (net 5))
 (segment (start 157.8864 96.8038) (end 166.7554 96.8038) (width 0.25) (layer "F.Cu") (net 16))
 (segment (start 166.7554 96.8038) (end 172.5168 102.5652) (width 0.25) (layer "F.Cu") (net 16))
 (segment (start 157.8864 94.2638) (end 167.7154 94.2638) (width 0.25) (layer "F.Cu") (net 17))
 (segment (start 167.7154 94.2638) (end 172.5168 99.0652) (width 0.25) (layer "F.Cu") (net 17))
 (segment (start 157.8864 91.7238) (end 168.6754 91.7238) (width 0.25) (layer "F.Cu") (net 18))
 (segment (start 168.6754 91.7238) (end 172.5168 95.5652) (width 0.25) (layer "F.Cu") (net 18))
 (segment (start 157.8864 89.1838) (end 169.6354 89.1838) (width 0.25) (layer "F.Cu") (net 19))
 (segment (start 169.6354 89.1838) (end 172.5168 92.0652) (width 0.25) (layer "F.Cu") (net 19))
 (segment (start 170.5954 86.6438) (end 172.5168 88.5652) (width 0.25) (layer "F.Cu") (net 20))
 (segment (start 157.8864 86.6438) (end 170.5954 86.6438) (width 0.25) (layer "F.Cu") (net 20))
 (segment (start 171.5554 84.1038) (end 172.5168 85.0652) (width 0.25) (layer "F.Cu") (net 21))
 (segment (start 157.8864 84.1038) (end 171.5554 84.1038) (width 0.25) (layer "F.Cu") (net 21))
 (segment (start 172.5168 81.5652) (end 157.8878 81.5652) (width 0.25) (layer "F.Cu") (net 22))
 (segment (start 157.8878 81.5652) (end 157.8864 81.5638) (width 0.25) (layer "F.Cu") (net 22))
 (segment (start 179.6288 70.0532) (end 176.1236 66.548) (width 0.25) (layer "F.Cu") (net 23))
 (segment (start 132.4864 79.0238) (end 139.2726 79.0238) (width 0.25) (layer "F.Cu") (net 23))
 (segment (start 179.6288 113.4872) (end 179.6288 70.0532) (width 0.25) (layer "F.Cu") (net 23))
 (segment (start 150.7236 90.4748) (end 150.7236 112.8776) (width 0.25) (layer "F.Cu") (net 23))
 (segment (start 178.2064 114.9096) (end 179.6288 113.4872) (width 0.25) (layer "F.Cu") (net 23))
 (segment (start 176.1236 66.548) (end 170.685 66.548) (width 0.25) (layer "F.Cu") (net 23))
 (segment (start 139.2726 79.0238) (end 150.7236 90.4748) (width 0.25) (layer "F.Cu") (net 23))
 (segment (start 152.7556 114.9096) (end 178.2064 114.9096) (width 0.25) (layer "F.Cu") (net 23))
 (segment (start 150.7236 112.8776) (end 152.7556 114.9096) (width 0.25) (layer "F.Cu") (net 23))
 (segment (start 170.685 64.008) (end 175.3616 64.008) (width 0.25) (layer "F.Cu") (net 24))
 (segment (start 152.5016 116.078) (end 149.0472 112.6236) (width 0.25) (layer "F.Cu") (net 24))
 (segment (start 144.9622 86.6438) (end 132.4864 86.6438) (width 0.25) (layer "F.Cu") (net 24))
 (segment (start 179.2224 116.078) (end 152.5016 116.078) (width 0.25) (layer "F.Cu") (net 24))
 (segment (start 149.1996 90.8812) (end 144.9622 86.6438) (width 0.25) (layer "F.Cu") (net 24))
 (segment (start 149.0472 91.0336) (end 149.1996 90.8812) (width 0.25) (layer "F.Cu") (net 24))
 (segment (start 149.0472 112.6236) (end 149.0472 91.0336) (width 0.25) (layer "F.Cu") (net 24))
 (segment (start 181.2544 114.046) (end 179.2224 116.078) (width 0.25) (layer "F.Cu") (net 24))
 (segment (start 175.3616 64.008) (end 181.2544 69.9008) (width 0.25) (layer "F.Cu") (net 24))
 (segment (start 181.2544 69.9008) (end 181.2544 114.046) (width 0.25) (layer "F.Cu") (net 24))
 (segment (start 177.8 112.2) (end 177.8 71.8) (width 0.25) (layer "F.Cu") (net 25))
 (segment (start 155.4 113.4) (end 176.6 113.4) (width 0.25) (layer "F.Cu") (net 25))
 (segment (start 177.8 71.8) (end 174.8 68.8) (width 0.25) (layer "F.Cu") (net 25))
 (segment (start 169.8 68.8) (end 168.2 67.2) (width 0.25) (layer "F.Cu") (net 25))
 (segment (start 168.2 67.2) (end 168.2 63.953) (width 0.25) (layer "F.Cu") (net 25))
 (segment (start 176.6 113.4) (end 177.8 112.2) (width 0.25) (layer "F.Cu") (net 25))
 (segment (start 137.3438 73.9438) (end 153.2 89.8) (width 0.25) (layer "F.Cu") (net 25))
 (segment (start 153.2 89.8) (end 153.2 111.2) (width 0.25) (layer "F.Cu") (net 25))
 (segment (start 153.2 111.2) (end 155.4 113.4) (width 0.25) (layer "F.Cu") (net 25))
 (segment (start 132.4864 73.9438) (end 137.3438 73.9438) (width 0.25) (layer "F.Cu") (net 25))
 (segment (start 168.2 63.953) (end 170.685 61.468) (width 0.25) (layer "F.Cu") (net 25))
 (segment (start 174.8 68.8) (end 169.8 68.8) (width 0.25) (layer "F.Cu") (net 25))
 (segment (start 165.7096 52.1197) (end 166.5213 51.308) (width 0.25) (layer "F.Cu") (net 15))
 (segment (start 166.5213 51.308) (end 170.685 51.308) (width 0.25) (layer "F.Cu") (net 15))
 (segment (start 114.105 83.305) (end 116.53 83.305) (width 0.25) (layer "F.Cu") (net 10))
 (segment (start 113.8 82.92) (end 113.8 83) (width 0.25) (layer "F.Cu") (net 10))
 (segment (start 113.8 83) (end 114.105 83.305) (width 0.25) (layer "F.Cu") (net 10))
 (segment (start 99 84.56) (end 109.2425 84.56) (width 0.25) (layer "F.Cu") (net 7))
 (segment (start 109.2425 84.56) (end 109.6025 84.2) (width 0.25) (layer "F.Cu") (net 7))
 (segment (start 106.5625 89.64) (end 109.6025 86.6) (width 0.25) (layer "F.Cu") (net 8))
 (segment (start 99 89.64) (end 106.5625 89.64) (width 0.25) (layer "F.Cu") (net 8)))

